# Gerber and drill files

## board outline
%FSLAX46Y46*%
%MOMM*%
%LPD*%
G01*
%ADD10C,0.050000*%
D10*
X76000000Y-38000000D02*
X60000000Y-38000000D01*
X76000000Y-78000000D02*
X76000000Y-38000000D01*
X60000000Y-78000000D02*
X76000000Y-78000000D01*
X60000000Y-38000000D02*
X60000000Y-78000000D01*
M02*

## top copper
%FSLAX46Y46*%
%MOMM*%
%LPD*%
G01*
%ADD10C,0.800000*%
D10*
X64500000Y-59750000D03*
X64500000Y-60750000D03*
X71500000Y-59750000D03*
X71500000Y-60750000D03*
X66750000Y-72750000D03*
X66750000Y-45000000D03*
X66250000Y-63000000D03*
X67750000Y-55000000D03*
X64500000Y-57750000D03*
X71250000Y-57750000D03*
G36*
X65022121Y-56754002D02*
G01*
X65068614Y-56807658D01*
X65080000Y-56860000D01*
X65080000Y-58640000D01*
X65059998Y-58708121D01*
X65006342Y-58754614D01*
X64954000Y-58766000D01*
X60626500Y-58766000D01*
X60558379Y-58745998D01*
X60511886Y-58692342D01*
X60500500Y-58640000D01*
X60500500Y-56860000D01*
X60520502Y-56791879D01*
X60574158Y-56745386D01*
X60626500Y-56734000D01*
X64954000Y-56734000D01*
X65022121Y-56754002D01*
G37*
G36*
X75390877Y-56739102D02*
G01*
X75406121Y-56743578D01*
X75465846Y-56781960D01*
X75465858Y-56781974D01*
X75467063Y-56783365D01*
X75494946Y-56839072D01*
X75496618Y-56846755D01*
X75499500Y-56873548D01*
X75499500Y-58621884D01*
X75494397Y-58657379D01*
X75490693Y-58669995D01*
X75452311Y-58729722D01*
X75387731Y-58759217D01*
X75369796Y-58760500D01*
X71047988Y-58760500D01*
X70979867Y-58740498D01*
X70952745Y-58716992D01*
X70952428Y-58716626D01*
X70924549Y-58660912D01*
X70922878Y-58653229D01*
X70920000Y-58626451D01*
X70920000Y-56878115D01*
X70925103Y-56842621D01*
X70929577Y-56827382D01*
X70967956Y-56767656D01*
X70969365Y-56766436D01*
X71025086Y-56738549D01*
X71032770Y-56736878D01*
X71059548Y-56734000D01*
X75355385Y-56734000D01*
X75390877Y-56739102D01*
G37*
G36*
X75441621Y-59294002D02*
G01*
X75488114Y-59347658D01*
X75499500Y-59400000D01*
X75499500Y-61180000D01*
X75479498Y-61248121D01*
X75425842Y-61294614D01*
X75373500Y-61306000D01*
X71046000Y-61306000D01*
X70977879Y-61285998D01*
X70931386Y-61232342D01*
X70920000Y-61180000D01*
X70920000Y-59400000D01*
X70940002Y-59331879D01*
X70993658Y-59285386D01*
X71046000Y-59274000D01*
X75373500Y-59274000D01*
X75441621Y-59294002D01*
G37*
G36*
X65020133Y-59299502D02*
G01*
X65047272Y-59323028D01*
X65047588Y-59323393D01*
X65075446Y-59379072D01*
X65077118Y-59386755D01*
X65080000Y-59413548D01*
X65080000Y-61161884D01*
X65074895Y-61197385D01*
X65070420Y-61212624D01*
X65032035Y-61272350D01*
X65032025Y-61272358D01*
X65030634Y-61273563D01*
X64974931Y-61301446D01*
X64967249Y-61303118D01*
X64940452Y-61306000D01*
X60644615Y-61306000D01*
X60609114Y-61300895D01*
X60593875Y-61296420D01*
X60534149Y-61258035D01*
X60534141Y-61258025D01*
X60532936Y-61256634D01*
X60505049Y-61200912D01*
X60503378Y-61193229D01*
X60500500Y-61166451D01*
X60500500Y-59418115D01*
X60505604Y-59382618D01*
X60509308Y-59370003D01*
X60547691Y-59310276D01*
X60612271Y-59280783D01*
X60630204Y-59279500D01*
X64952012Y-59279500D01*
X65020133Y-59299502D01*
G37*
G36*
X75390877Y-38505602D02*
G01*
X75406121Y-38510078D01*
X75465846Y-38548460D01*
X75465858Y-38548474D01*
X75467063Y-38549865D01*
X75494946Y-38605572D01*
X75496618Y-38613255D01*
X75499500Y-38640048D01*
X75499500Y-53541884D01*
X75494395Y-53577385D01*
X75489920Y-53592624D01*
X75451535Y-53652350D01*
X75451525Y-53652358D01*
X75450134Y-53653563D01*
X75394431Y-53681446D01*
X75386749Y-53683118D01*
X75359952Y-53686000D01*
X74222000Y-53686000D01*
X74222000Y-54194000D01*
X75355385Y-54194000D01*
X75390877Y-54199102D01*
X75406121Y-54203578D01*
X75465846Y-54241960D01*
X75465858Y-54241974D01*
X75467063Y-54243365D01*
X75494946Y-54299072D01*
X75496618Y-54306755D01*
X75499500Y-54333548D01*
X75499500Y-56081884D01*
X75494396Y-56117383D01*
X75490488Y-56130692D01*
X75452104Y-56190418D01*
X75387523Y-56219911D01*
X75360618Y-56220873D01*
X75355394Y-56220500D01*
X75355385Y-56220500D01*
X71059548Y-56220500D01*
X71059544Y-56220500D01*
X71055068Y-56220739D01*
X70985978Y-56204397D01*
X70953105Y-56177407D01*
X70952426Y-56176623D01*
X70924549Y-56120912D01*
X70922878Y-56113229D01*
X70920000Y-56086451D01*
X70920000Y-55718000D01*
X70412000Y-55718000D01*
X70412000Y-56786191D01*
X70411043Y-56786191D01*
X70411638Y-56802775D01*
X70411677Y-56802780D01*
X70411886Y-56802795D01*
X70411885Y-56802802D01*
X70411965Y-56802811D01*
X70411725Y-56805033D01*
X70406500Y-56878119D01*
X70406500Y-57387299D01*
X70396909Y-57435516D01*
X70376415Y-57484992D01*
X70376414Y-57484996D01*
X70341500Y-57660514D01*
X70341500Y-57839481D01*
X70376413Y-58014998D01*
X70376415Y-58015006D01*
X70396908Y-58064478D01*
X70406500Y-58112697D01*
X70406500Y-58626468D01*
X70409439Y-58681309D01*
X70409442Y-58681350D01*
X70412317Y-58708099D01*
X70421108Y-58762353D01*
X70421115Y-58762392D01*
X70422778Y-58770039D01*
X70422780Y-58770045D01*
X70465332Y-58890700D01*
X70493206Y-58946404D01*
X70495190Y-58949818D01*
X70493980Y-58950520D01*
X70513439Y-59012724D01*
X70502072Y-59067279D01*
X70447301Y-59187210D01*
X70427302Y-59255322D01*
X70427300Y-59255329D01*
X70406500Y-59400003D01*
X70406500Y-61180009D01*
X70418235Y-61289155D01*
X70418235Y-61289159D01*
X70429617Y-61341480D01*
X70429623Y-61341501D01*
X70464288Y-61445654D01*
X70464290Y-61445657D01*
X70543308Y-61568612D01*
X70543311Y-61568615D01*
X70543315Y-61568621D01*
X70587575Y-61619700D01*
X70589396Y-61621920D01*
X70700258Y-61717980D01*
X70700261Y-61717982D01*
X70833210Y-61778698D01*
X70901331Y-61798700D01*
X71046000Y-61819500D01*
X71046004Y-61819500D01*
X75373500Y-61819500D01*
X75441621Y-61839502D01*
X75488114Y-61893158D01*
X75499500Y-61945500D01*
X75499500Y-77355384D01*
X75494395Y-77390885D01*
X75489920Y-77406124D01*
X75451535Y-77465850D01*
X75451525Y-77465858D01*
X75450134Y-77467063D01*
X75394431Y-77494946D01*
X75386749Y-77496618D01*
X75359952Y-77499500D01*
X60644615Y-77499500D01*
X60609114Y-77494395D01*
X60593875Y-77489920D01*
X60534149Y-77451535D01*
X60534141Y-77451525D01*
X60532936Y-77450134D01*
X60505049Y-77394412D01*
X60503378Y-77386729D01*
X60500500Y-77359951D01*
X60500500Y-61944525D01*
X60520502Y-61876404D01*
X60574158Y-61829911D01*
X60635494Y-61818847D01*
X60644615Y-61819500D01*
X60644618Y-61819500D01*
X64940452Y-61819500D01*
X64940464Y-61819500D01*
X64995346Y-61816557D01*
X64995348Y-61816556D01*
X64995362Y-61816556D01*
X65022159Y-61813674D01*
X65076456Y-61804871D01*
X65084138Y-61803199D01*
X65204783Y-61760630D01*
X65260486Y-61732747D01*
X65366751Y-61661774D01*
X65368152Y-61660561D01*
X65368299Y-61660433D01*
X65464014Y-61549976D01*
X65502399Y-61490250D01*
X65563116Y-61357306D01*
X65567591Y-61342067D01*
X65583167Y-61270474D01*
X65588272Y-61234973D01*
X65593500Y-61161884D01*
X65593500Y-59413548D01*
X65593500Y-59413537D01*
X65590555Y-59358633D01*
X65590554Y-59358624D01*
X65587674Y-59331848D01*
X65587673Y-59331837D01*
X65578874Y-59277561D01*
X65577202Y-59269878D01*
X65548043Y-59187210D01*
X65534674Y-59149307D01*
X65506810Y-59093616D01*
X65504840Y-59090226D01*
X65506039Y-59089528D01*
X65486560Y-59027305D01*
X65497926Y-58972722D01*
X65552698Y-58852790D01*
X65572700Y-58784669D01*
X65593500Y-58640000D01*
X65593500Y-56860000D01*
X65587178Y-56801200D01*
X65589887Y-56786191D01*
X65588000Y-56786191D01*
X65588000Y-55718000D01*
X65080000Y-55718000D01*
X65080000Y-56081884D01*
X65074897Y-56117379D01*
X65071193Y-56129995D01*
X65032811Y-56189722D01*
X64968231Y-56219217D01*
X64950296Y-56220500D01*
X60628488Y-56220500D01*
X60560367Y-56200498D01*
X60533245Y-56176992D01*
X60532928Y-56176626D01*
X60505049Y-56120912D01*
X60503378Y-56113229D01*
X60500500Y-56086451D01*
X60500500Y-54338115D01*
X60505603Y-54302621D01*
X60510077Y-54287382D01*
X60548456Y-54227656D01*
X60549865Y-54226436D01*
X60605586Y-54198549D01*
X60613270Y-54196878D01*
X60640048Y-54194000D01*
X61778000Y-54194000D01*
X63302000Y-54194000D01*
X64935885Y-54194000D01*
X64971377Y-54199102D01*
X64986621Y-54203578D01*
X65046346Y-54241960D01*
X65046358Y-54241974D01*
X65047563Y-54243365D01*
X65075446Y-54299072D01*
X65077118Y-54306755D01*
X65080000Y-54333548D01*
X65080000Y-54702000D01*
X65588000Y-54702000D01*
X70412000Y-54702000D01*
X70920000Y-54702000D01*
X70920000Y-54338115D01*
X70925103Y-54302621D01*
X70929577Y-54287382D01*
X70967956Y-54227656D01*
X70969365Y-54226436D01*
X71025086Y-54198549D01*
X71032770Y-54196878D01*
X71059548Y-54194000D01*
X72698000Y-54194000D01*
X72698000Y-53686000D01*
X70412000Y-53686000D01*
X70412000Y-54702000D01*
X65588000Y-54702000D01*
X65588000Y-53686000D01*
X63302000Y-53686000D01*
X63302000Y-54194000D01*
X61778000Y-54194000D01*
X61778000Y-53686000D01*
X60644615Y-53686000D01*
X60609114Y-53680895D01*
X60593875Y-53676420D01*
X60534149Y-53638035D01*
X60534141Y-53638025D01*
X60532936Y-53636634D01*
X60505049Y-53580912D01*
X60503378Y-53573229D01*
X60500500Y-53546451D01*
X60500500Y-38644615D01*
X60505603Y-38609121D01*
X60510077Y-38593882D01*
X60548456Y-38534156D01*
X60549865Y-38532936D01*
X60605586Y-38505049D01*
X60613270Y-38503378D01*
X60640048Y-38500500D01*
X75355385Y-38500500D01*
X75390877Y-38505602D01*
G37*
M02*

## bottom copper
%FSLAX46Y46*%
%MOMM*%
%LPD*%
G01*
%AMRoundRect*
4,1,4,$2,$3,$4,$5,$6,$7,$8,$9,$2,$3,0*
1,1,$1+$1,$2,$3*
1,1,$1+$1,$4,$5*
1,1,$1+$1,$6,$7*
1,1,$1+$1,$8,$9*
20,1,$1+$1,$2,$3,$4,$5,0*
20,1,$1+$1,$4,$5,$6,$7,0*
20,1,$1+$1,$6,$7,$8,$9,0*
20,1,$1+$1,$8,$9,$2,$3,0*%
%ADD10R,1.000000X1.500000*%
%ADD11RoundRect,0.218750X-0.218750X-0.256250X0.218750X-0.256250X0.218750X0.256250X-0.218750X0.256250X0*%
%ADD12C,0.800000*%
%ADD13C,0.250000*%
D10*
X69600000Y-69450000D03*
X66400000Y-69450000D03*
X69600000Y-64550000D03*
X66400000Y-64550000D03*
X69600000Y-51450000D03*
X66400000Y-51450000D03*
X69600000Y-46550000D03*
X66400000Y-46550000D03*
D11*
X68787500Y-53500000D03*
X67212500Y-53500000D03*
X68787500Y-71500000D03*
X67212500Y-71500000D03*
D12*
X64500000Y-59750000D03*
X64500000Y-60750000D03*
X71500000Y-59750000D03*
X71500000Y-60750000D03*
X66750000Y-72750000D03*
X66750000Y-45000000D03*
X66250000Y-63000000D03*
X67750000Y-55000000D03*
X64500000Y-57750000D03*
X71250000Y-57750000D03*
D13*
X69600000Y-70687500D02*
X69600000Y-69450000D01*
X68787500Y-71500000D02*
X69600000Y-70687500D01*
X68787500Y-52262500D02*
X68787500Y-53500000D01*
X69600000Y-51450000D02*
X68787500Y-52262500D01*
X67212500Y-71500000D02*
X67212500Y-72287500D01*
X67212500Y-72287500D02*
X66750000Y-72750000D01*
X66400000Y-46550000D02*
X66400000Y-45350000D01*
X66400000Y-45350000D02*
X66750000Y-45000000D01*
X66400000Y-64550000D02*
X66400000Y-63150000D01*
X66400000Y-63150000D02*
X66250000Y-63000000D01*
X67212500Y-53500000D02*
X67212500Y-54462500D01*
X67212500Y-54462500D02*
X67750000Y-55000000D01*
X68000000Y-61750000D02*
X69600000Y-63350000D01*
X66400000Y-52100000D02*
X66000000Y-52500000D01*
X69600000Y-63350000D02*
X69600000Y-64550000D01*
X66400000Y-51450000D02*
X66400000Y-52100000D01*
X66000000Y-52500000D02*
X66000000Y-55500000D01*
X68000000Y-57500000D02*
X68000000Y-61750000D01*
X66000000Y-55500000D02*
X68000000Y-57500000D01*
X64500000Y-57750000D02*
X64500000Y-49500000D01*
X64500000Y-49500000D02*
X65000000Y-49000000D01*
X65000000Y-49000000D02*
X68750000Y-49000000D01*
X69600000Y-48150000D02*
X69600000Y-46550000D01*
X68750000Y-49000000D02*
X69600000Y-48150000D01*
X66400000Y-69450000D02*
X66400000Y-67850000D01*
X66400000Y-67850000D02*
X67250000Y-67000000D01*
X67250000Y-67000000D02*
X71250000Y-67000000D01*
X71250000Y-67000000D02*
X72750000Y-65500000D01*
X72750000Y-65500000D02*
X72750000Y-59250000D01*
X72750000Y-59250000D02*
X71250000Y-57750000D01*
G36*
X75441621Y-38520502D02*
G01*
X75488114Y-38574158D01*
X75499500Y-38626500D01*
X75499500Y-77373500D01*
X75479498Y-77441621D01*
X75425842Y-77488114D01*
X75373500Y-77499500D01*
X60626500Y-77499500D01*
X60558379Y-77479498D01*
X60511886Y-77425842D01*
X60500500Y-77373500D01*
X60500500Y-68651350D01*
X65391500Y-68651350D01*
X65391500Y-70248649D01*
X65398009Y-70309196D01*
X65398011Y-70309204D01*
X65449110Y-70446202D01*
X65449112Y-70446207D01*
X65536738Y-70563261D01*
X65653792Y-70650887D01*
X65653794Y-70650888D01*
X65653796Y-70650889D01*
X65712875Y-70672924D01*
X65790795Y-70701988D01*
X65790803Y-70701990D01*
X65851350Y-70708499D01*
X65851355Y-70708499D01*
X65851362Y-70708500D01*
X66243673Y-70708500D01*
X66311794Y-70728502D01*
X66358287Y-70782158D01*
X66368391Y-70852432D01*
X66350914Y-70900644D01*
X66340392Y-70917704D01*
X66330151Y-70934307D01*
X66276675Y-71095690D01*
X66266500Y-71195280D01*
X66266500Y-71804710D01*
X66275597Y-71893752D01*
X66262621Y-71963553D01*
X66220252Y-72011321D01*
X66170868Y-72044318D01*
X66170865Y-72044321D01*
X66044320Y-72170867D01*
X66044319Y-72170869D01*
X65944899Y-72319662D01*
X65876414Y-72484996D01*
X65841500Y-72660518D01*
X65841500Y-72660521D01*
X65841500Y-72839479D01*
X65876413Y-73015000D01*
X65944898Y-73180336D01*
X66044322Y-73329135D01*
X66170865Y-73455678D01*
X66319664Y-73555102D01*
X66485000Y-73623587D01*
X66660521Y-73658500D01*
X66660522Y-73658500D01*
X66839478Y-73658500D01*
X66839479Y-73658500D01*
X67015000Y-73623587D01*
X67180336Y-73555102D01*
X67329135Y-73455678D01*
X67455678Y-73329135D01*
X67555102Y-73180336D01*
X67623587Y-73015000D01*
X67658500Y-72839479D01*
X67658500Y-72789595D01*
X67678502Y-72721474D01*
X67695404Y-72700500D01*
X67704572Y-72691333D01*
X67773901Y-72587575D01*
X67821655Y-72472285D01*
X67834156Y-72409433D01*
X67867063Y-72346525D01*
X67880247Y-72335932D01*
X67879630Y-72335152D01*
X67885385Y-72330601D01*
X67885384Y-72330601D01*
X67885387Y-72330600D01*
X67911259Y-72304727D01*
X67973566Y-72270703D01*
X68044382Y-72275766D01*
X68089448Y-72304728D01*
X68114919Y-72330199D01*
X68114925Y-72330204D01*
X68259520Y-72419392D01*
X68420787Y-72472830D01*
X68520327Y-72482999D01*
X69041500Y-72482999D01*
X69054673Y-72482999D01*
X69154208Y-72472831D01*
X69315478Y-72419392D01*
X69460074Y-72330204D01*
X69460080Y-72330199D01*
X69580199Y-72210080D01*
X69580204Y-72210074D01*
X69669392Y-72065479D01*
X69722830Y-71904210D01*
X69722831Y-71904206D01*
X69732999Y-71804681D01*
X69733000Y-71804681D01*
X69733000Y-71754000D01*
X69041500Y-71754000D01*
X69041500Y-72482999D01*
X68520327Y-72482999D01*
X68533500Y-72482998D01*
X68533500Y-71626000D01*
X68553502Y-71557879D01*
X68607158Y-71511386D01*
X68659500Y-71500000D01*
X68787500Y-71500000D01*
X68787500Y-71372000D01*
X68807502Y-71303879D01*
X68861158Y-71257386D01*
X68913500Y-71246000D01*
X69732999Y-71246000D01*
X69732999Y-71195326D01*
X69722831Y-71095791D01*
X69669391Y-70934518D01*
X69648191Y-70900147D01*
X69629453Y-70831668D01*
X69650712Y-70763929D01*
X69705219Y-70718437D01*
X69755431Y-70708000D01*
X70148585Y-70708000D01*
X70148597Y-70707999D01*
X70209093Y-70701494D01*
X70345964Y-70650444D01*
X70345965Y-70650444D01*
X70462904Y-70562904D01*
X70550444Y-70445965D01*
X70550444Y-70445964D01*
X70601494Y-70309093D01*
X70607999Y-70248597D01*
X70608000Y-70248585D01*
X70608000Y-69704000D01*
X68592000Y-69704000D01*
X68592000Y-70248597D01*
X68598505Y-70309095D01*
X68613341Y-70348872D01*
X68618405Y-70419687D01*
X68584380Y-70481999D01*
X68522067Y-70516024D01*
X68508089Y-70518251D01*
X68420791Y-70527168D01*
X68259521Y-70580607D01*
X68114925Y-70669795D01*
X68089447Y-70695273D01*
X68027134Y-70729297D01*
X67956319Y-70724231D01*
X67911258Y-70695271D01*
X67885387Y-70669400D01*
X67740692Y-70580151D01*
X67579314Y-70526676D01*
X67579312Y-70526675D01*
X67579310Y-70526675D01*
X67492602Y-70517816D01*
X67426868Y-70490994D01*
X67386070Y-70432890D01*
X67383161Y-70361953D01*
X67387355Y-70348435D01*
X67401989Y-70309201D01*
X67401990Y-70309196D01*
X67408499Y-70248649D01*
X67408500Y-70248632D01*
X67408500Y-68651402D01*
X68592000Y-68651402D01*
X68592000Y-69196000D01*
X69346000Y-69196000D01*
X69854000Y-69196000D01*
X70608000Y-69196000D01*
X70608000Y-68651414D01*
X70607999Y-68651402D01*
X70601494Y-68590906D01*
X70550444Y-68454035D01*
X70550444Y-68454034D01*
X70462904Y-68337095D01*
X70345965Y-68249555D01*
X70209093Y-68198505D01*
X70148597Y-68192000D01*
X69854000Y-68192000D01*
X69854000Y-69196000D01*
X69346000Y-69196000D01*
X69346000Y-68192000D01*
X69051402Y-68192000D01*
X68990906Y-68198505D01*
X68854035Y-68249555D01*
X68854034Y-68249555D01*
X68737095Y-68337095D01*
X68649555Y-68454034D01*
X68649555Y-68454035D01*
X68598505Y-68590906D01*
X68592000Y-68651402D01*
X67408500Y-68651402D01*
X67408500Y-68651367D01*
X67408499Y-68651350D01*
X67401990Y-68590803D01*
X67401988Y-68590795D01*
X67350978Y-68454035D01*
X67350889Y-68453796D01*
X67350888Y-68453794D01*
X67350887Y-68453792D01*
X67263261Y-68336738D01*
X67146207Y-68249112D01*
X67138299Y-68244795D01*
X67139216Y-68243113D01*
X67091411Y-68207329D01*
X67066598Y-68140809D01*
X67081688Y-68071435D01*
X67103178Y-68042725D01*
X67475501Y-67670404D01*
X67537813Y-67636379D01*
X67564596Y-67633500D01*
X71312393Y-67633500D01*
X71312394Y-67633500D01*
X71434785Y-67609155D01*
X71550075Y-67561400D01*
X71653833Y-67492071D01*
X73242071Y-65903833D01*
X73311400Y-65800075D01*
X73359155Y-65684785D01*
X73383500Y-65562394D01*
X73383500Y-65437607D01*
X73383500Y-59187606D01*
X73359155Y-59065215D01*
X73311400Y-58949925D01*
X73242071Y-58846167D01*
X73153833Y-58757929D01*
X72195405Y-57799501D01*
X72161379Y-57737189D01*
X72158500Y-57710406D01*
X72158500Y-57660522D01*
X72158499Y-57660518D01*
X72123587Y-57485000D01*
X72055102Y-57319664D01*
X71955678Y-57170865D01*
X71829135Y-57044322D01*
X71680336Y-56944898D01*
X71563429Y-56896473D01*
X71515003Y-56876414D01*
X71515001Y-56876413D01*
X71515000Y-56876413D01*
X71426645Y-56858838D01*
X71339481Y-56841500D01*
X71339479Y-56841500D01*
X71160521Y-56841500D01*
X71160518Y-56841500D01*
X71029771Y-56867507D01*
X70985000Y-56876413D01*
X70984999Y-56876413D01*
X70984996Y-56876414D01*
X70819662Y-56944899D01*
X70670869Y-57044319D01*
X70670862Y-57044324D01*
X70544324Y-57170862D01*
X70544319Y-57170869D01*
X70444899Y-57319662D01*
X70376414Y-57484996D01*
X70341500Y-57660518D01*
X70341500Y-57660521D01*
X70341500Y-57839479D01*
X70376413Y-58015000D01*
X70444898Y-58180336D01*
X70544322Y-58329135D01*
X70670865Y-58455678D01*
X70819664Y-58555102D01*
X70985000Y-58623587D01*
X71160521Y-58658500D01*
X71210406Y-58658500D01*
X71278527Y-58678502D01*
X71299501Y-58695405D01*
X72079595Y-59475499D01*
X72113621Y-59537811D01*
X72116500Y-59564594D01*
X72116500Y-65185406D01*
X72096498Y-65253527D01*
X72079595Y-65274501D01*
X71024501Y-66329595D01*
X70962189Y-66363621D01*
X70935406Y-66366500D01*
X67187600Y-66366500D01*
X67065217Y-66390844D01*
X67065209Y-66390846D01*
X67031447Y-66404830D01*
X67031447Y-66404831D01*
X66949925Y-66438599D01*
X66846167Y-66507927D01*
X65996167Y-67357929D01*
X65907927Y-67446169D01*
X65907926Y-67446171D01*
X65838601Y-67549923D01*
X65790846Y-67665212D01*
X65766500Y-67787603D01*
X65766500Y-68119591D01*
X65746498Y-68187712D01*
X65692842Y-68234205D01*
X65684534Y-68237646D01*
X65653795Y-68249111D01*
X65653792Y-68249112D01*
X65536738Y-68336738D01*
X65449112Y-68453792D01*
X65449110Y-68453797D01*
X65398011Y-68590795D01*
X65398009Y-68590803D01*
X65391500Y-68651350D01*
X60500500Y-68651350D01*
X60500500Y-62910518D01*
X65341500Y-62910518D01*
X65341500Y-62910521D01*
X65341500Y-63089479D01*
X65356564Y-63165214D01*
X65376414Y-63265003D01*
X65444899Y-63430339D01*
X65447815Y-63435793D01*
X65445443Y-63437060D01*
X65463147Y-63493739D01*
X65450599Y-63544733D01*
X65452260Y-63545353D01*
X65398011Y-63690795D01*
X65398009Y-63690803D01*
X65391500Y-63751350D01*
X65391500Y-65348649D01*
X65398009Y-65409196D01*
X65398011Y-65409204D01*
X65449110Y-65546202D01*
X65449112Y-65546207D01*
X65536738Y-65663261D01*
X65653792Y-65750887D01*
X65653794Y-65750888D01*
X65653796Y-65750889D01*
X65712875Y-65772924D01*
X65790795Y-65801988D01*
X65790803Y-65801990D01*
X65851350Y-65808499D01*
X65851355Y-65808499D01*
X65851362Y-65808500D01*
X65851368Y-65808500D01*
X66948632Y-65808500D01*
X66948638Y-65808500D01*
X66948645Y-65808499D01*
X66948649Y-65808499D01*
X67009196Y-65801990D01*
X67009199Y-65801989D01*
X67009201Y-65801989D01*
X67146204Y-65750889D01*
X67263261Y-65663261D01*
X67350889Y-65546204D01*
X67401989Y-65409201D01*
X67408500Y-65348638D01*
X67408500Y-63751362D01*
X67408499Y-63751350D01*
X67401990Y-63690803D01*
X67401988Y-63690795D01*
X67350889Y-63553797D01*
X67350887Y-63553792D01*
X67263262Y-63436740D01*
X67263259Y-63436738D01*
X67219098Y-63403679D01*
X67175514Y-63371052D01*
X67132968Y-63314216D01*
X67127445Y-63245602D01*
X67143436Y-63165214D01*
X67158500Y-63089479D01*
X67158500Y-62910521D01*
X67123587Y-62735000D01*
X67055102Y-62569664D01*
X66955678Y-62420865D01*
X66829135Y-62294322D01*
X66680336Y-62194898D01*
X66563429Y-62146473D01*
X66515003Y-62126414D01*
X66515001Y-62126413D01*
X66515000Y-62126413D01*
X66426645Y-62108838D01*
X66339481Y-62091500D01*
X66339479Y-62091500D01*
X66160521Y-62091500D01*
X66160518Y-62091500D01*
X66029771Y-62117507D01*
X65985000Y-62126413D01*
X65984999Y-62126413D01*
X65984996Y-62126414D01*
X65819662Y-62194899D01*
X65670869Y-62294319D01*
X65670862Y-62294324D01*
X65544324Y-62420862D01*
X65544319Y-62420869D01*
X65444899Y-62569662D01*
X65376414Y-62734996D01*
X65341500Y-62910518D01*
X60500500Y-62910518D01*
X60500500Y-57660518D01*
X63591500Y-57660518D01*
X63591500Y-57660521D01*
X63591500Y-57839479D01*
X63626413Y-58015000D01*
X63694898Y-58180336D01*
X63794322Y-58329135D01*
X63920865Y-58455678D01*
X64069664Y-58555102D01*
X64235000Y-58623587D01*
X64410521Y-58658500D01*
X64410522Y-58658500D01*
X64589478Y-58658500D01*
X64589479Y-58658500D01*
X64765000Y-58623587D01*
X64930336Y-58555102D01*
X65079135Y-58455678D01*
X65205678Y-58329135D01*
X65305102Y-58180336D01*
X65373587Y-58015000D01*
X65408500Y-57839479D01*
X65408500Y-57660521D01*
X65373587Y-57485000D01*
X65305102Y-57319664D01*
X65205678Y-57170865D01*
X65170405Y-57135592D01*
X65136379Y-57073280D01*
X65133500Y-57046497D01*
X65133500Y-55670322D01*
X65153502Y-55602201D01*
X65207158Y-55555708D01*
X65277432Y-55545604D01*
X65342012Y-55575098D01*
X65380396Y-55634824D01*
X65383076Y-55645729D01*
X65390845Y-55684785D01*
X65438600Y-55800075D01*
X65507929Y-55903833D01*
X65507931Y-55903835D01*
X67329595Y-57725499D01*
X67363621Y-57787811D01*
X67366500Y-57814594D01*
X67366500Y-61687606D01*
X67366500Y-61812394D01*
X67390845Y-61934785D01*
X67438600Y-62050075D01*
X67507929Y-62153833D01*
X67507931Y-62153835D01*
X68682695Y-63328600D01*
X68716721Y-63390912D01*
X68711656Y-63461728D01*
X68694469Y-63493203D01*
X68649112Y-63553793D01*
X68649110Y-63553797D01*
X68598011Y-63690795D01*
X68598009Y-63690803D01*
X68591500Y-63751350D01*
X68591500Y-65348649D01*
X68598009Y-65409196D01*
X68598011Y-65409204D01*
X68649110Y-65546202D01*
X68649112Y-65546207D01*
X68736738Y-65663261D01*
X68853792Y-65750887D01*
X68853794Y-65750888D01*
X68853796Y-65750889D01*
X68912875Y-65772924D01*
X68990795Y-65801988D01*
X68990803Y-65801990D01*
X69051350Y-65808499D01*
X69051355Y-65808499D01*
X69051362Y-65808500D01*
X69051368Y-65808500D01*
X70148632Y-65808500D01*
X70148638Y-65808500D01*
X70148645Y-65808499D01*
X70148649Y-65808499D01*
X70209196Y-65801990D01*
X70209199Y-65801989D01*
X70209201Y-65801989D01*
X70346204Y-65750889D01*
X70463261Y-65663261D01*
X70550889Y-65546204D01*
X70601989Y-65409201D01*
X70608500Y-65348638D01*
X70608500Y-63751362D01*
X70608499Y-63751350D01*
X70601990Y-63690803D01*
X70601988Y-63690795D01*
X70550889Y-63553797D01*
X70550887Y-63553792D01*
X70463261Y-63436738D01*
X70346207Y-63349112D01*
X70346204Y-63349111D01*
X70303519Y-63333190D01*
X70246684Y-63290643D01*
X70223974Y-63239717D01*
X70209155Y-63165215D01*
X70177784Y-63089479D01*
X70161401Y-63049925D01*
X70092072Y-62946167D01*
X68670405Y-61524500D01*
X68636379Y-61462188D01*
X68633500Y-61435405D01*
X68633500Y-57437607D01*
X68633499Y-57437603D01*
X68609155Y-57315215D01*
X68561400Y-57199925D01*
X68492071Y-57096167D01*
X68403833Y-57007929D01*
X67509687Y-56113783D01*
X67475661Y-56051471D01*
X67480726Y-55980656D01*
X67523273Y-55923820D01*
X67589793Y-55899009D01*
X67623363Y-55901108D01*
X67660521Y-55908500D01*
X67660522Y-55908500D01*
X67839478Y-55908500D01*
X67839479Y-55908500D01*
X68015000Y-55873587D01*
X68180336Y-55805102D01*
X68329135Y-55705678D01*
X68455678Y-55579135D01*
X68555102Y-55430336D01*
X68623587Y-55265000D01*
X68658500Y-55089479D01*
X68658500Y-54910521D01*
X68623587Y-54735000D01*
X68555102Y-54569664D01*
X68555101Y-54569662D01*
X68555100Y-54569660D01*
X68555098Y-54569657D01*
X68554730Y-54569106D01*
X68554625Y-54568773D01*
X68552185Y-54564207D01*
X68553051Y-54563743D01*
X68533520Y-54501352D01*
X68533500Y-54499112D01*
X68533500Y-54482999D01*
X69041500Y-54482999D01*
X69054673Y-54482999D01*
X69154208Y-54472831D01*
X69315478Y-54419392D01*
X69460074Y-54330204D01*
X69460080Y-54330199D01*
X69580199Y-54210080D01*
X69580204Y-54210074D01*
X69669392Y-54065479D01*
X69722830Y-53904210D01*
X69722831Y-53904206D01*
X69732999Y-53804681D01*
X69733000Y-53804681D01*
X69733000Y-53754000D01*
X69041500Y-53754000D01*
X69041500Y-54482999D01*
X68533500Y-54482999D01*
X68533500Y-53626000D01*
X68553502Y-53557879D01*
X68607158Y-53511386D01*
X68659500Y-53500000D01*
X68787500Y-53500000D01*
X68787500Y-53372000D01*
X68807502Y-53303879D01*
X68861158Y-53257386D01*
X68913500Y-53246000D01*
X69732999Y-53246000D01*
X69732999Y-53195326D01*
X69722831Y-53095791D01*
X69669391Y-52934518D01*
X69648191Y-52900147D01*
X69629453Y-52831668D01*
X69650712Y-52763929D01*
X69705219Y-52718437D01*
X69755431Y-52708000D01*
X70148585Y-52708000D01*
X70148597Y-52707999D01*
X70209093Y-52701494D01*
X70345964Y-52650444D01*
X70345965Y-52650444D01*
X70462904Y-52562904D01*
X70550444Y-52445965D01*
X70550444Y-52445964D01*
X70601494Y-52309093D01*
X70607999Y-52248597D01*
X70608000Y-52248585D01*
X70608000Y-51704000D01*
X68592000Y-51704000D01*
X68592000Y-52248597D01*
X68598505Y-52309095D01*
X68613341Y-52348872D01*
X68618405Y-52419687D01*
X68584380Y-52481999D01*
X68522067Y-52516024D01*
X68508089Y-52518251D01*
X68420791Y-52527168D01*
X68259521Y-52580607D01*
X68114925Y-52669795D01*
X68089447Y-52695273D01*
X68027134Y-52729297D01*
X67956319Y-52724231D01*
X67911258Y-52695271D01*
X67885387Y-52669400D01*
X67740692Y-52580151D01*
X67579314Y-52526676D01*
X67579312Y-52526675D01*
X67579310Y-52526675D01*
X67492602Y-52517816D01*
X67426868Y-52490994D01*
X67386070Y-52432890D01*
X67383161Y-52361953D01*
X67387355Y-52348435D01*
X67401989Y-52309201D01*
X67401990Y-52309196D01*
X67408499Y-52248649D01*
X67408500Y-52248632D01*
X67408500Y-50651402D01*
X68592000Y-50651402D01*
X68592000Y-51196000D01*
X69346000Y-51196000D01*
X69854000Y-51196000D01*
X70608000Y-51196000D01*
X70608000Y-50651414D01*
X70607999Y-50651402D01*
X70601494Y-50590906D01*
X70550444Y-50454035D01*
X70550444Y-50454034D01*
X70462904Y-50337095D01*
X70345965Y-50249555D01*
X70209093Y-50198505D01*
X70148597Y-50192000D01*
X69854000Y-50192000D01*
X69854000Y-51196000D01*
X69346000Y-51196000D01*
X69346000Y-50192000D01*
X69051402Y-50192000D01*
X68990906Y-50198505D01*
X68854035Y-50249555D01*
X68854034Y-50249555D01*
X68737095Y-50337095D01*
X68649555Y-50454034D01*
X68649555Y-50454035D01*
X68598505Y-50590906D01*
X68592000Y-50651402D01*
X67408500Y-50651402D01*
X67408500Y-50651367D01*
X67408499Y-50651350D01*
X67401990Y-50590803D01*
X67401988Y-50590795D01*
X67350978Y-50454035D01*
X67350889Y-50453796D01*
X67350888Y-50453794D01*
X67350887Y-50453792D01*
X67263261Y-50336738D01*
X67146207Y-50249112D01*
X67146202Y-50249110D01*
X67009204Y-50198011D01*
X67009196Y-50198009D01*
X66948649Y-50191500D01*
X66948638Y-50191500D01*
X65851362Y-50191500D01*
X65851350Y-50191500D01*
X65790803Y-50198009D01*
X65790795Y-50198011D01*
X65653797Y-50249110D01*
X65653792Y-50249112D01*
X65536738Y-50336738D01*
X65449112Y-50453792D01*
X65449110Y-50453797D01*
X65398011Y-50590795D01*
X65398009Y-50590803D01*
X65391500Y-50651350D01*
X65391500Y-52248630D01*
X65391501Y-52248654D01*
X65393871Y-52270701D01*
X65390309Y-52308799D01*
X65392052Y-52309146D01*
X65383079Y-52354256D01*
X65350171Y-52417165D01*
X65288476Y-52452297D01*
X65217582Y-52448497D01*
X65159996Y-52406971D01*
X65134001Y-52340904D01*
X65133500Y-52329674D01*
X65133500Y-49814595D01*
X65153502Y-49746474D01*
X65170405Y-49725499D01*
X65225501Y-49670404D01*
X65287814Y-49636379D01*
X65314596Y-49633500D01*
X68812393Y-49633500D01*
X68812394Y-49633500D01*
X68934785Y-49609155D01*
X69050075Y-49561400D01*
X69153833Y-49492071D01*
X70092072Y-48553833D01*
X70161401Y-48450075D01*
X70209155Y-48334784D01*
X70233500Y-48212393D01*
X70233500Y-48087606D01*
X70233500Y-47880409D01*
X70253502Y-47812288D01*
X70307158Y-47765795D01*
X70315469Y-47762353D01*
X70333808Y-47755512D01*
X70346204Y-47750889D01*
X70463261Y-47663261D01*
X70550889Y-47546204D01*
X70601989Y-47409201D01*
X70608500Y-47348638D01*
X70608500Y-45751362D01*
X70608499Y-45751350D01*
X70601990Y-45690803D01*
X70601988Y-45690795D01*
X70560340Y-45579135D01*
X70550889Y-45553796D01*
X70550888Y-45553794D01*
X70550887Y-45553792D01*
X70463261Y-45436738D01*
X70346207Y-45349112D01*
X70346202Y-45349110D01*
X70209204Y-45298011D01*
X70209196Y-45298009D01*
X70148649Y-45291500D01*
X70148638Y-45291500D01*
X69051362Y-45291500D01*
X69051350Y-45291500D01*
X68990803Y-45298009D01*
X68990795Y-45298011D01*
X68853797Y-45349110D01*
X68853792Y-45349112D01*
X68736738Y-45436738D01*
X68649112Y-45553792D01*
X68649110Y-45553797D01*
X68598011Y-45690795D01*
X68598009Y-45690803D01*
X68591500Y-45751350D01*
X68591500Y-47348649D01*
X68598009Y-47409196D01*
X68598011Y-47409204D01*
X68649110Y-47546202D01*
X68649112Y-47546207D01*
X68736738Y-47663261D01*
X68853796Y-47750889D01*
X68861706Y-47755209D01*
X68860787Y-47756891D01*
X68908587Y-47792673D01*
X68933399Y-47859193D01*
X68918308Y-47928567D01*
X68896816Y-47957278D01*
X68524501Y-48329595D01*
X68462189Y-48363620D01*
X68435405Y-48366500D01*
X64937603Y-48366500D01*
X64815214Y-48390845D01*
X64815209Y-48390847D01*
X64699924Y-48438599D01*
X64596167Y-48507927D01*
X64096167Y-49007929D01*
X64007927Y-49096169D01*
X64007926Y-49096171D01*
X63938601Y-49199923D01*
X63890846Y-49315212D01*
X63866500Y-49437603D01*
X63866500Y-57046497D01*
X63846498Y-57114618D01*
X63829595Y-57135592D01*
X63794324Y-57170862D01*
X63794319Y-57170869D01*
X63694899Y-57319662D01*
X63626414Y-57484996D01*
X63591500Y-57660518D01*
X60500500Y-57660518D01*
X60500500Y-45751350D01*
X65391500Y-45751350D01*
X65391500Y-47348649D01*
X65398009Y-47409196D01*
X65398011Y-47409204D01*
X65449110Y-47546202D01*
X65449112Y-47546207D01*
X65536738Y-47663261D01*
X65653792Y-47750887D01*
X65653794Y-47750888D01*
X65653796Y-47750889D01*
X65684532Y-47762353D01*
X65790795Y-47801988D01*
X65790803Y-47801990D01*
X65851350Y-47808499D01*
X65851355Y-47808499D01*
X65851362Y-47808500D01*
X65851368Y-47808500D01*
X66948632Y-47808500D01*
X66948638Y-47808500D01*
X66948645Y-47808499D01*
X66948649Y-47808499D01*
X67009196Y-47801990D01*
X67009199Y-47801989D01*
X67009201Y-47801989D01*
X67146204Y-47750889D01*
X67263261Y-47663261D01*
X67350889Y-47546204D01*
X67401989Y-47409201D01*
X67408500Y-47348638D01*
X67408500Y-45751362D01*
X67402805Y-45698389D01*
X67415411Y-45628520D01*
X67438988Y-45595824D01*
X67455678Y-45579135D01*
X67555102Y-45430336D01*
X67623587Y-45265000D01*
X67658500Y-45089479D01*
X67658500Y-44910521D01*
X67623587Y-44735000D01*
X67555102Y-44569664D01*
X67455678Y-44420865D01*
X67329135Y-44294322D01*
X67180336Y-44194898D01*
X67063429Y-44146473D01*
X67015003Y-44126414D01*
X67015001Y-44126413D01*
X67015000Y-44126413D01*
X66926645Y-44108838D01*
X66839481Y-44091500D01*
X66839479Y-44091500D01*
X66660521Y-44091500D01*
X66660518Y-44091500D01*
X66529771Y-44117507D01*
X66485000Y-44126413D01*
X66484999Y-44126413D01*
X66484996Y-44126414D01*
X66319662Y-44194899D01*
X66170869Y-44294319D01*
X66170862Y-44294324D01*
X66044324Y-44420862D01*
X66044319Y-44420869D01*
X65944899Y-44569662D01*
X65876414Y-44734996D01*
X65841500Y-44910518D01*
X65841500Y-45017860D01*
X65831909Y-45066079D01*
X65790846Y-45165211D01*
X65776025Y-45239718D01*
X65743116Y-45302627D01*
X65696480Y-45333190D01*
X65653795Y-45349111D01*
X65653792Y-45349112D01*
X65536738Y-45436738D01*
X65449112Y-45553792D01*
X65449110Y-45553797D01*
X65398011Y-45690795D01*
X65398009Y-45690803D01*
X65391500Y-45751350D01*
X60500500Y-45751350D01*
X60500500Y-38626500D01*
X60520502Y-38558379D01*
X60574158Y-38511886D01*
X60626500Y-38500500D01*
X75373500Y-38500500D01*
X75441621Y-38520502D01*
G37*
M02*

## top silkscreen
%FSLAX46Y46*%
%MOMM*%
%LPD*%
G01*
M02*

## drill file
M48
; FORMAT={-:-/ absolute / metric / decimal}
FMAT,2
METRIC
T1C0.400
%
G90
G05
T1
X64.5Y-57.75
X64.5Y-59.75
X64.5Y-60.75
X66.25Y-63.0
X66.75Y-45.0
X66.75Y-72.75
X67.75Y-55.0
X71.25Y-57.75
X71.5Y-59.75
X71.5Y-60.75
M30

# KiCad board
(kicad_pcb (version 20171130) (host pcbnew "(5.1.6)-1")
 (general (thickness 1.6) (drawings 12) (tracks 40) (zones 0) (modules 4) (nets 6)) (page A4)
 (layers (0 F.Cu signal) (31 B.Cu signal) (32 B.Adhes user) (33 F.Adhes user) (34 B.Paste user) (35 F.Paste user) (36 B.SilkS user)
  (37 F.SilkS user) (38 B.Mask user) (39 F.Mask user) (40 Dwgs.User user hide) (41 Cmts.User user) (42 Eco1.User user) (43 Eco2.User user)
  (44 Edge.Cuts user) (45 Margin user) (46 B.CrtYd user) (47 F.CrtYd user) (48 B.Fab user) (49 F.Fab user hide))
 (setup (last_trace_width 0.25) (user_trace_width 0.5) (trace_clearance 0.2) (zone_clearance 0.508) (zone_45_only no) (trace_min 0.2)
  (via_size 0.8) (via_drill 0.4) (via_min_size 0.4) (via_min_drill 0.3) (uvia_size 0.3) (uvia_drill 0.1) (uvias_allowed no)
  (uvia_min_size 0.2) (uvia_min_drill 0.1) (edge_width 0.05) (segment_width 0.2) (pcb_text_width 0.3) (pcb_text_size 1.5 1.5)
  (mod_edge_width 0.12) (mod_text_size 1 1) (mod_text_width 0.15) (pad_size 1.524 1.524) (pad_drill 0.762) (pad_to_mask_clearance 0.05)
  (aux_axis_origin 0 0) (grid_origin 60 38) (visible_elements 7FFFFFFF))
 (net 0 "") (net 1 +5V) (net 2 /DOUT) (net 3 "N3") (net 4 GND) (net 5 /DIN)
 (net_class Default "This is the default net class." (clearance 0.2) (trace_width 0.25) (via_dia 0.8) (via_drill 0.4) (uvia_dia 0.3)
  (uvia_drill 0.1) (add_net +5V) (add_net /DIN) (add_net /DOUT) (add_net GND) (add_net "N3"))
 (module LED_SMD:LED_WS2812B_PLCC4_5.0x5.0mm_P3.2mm (layer B.Cu) (at 68 67 90)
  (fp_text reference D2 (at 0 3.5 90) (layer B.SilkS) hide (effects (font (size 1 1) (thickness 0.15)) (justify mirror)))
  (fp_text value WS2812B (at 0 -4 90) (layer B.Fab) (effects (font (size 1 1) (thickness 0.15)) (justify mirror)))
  (pad 1 smd rect (at -2.45 1.6 90) (size 1.5 1) (layers B.Cu B.Paste B.Mask) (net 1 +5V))
  (pad 2 smd rect (at -2.45 -1.6 90) (size 1.5 1) (layers B.Cu B.Paste B.Mask) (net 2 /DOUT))
  (pad 4 smd rect (at 2.45 1.6 90) (size 1.5 1) (layers B.Cu B.Paste B.Mask) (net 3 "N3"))
  (pad 3 smd rect (at 2.45 -1.6 90) (size 1.5 1) (layers B.Cu B.Paste B.Mask) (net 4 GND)))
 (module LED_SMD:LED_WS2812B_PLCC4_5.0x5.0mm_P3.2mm (layer B.Cu) (at 68 49 90)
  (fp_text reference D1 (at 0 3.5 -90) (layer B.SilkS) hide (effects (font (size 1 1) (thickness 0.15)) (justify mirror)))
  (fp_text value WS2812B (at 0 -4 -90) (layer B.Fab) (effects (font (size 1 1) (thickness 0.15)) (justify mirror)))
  (pad 1 smd rect (at -2.45 1.6 90) (size 1.5 1) (layers B.Cu B.Paste B.Mask) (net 1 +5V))
  (pad 2 smd rect (at -2.45 -1.6 90) (size 1.5 1) (layers B.Cu B.Paste B.Mask) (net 3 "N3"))
  (pad 4 smd rect (at 2.45 1.6 90) (size 1.5 1) (layers B.Cu B.Paste B.Mask) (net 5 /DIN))
  (pad 3 smd rect (at 2.45 -1.6 90) (size 1.5 1) (layers B.Cu B.Paste B.Mask) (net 4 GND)))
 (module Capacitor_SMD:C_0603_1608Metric (layer B.Cu) (at 68 53.5)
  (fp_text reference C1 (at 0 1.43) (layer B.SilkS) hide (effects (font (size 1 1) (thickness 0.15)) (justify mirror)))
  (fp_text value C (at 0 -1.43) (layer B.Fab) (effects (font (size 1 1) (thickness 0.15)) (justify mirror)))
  (pad 2 smd roundrect (at 0.7875 0) (size 0.875 0.95) (layers B.Cu B.Paste B.Mask) (roundrect_rratio 0.25) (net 1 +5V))
  (pad 1 smd roundrect (at -0.7875 0) (size 0.875 0.95) (layers B.Cu B.Paste B.Mask) (roundrect_rratio 0.25) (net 4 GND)))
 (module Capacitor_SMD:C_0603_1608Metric (layer B.Cu) (at 68 71.5)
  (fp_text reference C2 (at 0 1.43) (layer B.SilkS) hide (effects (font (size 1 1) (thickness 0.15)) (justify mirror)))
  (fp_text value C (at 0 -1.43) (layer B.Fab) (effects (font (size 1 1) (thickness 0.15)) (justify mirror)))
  (pad 2 smd roundrect (at 0.7875 0) (size 0.875 0.95) (layers B.Cu B.Paste B.Mask) (roundrect_rratio 0.25) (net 1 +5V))
  (pad 1 smd roundrect (at -0.7875 0) (size 0.875 0.95) (layers B.Cu B.Paste B.Mask) (roundrect_rratio 0.25) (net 4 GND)))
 (gr_line (start 76 38) (end 60 38) (layer Edge.Cuts) (width 0.05))
 (gr_line (start 76 78) (end 76 38) (layer Edge.Cuts) (width 0.05))
 (gr_line (start 60 78) (end 76 78) (layer Edge.Cuts) (width 0.05))
 (gr_line (start 60 38) (end 60 78) (layer Edge.Cuts) (width 0.05))
 (via (at 64.5 59.75) (size 0.8) (drill 0.4) (layers F.Cu B.Cu) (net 1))
 (via (at 64.5 60.75) (size 0.8) (drill 0.4) (layers F.Cu B.Cu) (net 1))
 (via (at 71.5 59.75) (size 0.8) (drill 0.4) (layers F.Cu B.Cu) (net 1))
 (via (at 71.5 60.75) (size 0.8) (drill 0.4) (layers F.Cu B.Cu) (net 1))
 (segment (start 69.6 70.6875) (end 69.6 69.45) (width 0.25) (layer B.Cu) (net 1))
 (segment (start 68.7875 71.5) (end 69.6 70.6875) (width 0.25) (layer B.Cu) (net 1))
 (segment (start 68.7875 52.2625) (end 68.7875 53.5) (width 0.25) (layer B.Cu) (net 1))
 (segment (start 69.6 51.45) (end 68.7875 52.2625) (width 0.25) (layer B.Cu) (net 1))
 (via (at 66.75 72.75) (size 0.8) (drill 0.4) (layers F.Cu B.Cu) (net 4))
 (segment (start 67.2125 71.5) (end 67.2125 72.2875) (width 0.25) (layer B.Cu) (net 4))
 (segment (start 67.2125 72.2875) (end 66.75 72.75) (width 0.25) (layer B.Cu) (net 4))
 (via (at 66.75 45) (size 0.8) (drill 0.4) (layers F.Cu B.Cu) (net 4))
 (segment (start 66.4 46.55) (end 66.4 45.35) (width 0.25) (layer B.Cu) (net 4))
 (segment (start 66.4 45.35) (end 66.75 45) (width 0.25) (layer B.Cu) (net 4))
 (via (at 66.25 63) (size 0.8) (drill 0.4) (layers F.Cu B.Cu) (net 4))
 (segment (start 66.4 64.55) (end 66.4 63.15) (width 0.25) (layer B.Cu) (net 4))
 (segment (start 66.4 63.15) (end 66.25 63) (width 0.25) (layer B.Cu) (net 4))
 (via (at 67.75 55) (size 0.8) (drill 0.4) (layers F.Cu B.Cu) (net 4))
 (segment (start 67.2125 53.5) (end 67.2125 54.4625) (width 0.25) (layer B.Cu) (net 4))
 (segment (start 67.2125 54.4625) (end 67.75 55) (width 0.25) (layer B.Cu) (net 4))
 (segment (start 68 61.75) (end 69.6 63.35) (width 0.25) (layer B.Cu) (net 3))
 (segment (start 66.4 52.1) (end 66 52.5) (width 0.25) (layer B.Cu) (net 3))
 (segment (start 69.6 63.35) (end 69.6 64.55) (width 0.25) (layer B.Cu) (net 3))
 (segment (start 66.4 51.45) (end 66.4 52.1) (width 0.25) (layer B.Cu) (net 3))
 (segment (start 66 52.5) (end 66 55.5) (width 0.25) (layer B.Cu) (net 3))
 (segment (start 68 57.5) (end 68 61.75) (width 0.25) (layer B.Cu) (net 3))
 (segment (start 66 55.5) (end 68 57.5) (width 0.25) (layer B.Cu) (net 3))
 (via (at 64.5 57.75) (size 0.8) (drill 0.4) (layers F.Cu B.Cu) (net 5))
 (segment (start 64.5 57.75) (end 64.5 49.5) (width 0.25) (layer B.Cu) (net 5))
 (segment (start 64.5 49.5) (end 65 49) (width 0.25) (layer B.Cu) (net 5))
 (segment (start 65 49) (end 68.75 49) (width 0.25) (layer B.Cu) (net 5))
 (segment (start 69.6 48.15) (end 69.6 46.55) (width 0.25) (layer B.Cu) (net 5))
 (segment (start 68.75 49) (end 69.6 48.15) (width 0.25) (layer B.Cu) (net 5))
 (segment (start 66.4 69.45) (end 66.4 67.85) (width 0.25) (layer B.Cu) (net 2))
 (segment (start 66.4 67.85) (end 67.25 67) (width 0.25) (layer B.Cu) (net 2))
 (segment (start 67.25 67) (end 71.25 67) (width 0.25) (layer B.Cu) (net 2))
 (segment (start 71.25 67) (end 72.75 65.5) (width 0.25) (layer B.Cu) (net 2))
 (segment (start 72.75 65.5) (end 72.75 59.25) (width 0.25) (layer B.Cu) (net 2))
 (segment (start 72.75 59.25) (end 71.25 57.75) (width 0.25) (layer B.Cu) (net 2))
 (via (at 71.25 57.75) (size 0.8) (drill 0.4) (layers F.Cu B.Cu) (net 2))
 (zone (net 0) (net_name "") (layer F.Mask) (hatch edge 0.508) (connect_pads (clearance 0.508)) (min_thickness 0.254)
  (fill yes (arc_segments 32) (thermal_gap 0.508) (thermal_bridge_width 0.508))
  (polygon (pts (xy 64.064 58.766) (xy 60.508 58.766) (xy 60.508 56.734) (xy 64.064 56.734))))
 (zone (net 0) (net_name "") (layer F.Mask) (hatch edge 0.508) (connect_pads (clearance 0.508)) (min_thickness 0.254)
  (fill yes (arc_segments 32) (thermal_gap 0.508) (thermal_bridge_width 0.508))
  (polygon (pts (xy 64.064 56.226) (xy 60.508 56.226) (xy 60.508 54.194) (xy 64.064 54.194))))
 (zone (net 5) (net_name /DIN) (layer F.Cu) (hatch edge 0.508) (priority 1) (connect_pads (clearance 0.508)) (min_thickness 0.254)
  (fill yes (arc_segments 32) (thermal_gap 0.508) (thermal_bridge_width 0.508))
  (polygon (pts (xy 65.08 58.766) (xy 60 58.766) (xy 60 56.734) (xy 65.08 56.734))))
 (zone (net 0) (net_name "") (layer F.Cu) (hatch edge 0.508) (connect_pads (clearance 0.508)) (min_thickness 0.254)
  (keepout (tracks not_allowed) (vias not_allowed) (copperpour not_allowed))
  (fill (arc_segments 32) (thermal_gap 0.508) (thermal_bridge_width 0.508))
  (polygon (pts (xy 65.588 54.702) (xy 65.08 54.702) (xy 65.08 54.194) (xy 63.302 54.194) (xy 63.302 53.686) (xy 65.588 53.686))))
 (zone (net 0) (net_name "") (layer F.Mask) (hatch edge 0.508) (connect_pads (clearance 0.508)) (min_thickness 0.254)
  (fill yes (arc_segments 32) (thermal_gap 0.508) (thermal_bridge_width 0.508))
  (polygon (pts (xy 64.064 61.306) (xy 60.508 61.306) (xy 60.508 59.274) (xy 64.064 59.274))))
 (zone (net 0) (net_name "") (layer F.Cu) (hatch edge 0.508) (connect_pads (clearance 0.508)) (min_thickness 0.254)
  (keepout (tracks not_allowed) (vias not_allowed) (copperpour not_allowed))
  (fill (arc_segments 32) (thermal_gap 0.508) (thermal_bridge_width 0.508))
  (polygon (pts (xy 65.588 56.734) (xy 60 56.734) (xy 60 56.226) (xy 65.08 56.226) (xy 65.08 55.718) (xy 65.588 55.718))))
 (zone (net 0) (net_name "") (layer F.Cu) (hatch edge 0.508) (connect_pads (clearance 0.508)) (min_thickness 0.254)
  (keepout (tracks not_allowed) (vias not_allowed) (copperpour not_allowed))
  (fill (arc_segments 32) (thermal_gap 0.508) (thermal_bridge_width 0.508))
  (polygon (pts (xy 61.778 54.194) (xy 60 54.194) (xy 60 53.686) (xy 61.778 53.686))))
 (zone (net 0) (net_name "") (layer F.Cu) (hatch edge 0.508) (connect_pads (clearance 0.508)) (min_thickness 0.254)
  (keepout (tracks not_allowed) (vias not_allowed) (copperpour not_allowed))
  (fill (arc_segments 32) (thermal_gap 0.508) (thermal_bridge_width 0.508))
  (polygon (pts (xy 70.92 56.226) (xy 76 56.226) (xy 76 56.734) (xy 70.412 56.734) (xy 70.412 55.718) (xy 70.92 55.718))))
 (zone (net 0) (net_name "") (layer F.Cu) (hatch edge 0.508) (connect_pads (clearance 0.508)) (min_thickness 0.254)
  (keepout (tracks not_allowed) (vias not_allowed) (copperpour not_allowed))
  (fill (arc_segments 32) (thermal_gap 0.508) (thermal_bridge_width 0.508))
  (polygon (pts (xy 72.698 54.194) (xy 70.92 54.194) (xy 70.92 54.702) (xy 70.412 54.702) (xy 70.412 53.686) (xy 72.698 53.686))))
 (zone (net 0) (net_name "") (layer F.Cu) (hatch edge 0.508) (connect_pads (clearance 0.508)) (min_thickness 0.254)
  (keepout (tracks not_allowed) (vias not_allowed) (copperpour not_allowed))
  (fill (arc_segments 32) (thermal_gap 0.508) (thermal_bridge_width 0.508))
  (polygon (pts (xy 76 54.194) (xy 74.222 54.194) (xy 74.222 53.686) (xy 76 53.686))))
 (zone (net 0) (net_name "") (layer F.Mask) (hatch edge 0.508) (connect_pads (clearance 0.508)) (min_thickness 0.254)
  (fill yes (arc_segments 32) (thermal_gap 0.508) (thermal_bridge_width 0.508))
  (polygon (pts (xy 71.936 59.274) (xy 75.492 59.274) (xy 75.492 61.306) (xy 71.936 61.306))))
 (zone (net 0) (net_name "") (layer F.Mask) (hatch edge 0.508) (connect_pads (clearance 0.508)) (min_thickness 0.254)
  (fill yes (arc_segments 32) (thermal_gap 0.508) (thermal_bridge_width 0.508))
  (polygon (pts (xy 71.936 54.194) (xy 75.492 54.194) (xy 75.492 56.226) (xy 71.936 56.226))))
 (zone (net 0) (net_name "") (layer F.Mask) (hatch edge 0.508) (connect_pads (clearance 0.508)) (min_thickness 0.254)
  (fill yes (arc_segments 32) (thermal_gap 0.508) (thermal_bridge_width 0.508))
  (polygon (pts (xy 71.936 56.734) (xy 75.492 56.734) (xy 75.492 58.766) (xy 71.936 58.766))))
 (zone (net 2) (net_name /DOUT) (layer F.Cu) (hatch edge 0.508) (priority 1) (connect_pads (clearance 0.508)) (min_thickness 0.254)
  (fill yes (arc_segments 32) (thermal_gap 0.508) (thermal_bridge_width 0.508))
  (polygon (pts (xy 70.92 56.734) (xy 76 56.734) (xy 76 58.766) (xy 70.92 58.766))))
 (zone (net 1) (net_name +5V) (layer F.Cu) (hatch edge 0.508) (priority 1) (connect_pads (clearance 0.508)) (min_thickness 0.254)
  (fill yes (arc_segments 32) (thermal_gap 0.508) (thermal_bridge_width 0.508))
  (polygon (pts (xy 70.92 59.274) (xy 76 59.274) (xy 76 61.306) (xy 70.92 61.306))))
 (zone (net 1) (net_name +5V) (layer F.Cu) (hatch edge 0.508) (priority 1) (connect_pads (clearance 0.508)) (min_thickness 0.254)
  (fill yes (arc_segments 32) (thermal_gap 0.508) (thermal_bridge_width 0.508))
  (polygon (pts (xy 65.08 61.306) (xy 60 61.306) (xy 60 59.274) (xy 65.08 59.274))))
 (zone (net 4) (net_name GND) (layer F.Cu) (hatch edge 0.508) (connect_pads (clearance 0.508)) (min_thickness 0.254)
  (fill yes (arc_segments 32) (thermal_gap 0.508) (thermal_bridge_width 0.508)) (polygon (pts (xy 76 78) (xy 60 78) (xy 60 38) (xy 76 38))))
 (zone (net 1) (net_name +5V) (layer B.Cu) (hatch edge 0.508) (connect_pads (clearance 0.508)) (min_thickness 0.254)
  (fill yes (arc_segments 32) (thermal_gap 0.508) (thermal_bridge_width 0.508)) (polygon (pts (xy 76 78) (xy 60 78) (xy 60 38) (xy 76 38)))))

